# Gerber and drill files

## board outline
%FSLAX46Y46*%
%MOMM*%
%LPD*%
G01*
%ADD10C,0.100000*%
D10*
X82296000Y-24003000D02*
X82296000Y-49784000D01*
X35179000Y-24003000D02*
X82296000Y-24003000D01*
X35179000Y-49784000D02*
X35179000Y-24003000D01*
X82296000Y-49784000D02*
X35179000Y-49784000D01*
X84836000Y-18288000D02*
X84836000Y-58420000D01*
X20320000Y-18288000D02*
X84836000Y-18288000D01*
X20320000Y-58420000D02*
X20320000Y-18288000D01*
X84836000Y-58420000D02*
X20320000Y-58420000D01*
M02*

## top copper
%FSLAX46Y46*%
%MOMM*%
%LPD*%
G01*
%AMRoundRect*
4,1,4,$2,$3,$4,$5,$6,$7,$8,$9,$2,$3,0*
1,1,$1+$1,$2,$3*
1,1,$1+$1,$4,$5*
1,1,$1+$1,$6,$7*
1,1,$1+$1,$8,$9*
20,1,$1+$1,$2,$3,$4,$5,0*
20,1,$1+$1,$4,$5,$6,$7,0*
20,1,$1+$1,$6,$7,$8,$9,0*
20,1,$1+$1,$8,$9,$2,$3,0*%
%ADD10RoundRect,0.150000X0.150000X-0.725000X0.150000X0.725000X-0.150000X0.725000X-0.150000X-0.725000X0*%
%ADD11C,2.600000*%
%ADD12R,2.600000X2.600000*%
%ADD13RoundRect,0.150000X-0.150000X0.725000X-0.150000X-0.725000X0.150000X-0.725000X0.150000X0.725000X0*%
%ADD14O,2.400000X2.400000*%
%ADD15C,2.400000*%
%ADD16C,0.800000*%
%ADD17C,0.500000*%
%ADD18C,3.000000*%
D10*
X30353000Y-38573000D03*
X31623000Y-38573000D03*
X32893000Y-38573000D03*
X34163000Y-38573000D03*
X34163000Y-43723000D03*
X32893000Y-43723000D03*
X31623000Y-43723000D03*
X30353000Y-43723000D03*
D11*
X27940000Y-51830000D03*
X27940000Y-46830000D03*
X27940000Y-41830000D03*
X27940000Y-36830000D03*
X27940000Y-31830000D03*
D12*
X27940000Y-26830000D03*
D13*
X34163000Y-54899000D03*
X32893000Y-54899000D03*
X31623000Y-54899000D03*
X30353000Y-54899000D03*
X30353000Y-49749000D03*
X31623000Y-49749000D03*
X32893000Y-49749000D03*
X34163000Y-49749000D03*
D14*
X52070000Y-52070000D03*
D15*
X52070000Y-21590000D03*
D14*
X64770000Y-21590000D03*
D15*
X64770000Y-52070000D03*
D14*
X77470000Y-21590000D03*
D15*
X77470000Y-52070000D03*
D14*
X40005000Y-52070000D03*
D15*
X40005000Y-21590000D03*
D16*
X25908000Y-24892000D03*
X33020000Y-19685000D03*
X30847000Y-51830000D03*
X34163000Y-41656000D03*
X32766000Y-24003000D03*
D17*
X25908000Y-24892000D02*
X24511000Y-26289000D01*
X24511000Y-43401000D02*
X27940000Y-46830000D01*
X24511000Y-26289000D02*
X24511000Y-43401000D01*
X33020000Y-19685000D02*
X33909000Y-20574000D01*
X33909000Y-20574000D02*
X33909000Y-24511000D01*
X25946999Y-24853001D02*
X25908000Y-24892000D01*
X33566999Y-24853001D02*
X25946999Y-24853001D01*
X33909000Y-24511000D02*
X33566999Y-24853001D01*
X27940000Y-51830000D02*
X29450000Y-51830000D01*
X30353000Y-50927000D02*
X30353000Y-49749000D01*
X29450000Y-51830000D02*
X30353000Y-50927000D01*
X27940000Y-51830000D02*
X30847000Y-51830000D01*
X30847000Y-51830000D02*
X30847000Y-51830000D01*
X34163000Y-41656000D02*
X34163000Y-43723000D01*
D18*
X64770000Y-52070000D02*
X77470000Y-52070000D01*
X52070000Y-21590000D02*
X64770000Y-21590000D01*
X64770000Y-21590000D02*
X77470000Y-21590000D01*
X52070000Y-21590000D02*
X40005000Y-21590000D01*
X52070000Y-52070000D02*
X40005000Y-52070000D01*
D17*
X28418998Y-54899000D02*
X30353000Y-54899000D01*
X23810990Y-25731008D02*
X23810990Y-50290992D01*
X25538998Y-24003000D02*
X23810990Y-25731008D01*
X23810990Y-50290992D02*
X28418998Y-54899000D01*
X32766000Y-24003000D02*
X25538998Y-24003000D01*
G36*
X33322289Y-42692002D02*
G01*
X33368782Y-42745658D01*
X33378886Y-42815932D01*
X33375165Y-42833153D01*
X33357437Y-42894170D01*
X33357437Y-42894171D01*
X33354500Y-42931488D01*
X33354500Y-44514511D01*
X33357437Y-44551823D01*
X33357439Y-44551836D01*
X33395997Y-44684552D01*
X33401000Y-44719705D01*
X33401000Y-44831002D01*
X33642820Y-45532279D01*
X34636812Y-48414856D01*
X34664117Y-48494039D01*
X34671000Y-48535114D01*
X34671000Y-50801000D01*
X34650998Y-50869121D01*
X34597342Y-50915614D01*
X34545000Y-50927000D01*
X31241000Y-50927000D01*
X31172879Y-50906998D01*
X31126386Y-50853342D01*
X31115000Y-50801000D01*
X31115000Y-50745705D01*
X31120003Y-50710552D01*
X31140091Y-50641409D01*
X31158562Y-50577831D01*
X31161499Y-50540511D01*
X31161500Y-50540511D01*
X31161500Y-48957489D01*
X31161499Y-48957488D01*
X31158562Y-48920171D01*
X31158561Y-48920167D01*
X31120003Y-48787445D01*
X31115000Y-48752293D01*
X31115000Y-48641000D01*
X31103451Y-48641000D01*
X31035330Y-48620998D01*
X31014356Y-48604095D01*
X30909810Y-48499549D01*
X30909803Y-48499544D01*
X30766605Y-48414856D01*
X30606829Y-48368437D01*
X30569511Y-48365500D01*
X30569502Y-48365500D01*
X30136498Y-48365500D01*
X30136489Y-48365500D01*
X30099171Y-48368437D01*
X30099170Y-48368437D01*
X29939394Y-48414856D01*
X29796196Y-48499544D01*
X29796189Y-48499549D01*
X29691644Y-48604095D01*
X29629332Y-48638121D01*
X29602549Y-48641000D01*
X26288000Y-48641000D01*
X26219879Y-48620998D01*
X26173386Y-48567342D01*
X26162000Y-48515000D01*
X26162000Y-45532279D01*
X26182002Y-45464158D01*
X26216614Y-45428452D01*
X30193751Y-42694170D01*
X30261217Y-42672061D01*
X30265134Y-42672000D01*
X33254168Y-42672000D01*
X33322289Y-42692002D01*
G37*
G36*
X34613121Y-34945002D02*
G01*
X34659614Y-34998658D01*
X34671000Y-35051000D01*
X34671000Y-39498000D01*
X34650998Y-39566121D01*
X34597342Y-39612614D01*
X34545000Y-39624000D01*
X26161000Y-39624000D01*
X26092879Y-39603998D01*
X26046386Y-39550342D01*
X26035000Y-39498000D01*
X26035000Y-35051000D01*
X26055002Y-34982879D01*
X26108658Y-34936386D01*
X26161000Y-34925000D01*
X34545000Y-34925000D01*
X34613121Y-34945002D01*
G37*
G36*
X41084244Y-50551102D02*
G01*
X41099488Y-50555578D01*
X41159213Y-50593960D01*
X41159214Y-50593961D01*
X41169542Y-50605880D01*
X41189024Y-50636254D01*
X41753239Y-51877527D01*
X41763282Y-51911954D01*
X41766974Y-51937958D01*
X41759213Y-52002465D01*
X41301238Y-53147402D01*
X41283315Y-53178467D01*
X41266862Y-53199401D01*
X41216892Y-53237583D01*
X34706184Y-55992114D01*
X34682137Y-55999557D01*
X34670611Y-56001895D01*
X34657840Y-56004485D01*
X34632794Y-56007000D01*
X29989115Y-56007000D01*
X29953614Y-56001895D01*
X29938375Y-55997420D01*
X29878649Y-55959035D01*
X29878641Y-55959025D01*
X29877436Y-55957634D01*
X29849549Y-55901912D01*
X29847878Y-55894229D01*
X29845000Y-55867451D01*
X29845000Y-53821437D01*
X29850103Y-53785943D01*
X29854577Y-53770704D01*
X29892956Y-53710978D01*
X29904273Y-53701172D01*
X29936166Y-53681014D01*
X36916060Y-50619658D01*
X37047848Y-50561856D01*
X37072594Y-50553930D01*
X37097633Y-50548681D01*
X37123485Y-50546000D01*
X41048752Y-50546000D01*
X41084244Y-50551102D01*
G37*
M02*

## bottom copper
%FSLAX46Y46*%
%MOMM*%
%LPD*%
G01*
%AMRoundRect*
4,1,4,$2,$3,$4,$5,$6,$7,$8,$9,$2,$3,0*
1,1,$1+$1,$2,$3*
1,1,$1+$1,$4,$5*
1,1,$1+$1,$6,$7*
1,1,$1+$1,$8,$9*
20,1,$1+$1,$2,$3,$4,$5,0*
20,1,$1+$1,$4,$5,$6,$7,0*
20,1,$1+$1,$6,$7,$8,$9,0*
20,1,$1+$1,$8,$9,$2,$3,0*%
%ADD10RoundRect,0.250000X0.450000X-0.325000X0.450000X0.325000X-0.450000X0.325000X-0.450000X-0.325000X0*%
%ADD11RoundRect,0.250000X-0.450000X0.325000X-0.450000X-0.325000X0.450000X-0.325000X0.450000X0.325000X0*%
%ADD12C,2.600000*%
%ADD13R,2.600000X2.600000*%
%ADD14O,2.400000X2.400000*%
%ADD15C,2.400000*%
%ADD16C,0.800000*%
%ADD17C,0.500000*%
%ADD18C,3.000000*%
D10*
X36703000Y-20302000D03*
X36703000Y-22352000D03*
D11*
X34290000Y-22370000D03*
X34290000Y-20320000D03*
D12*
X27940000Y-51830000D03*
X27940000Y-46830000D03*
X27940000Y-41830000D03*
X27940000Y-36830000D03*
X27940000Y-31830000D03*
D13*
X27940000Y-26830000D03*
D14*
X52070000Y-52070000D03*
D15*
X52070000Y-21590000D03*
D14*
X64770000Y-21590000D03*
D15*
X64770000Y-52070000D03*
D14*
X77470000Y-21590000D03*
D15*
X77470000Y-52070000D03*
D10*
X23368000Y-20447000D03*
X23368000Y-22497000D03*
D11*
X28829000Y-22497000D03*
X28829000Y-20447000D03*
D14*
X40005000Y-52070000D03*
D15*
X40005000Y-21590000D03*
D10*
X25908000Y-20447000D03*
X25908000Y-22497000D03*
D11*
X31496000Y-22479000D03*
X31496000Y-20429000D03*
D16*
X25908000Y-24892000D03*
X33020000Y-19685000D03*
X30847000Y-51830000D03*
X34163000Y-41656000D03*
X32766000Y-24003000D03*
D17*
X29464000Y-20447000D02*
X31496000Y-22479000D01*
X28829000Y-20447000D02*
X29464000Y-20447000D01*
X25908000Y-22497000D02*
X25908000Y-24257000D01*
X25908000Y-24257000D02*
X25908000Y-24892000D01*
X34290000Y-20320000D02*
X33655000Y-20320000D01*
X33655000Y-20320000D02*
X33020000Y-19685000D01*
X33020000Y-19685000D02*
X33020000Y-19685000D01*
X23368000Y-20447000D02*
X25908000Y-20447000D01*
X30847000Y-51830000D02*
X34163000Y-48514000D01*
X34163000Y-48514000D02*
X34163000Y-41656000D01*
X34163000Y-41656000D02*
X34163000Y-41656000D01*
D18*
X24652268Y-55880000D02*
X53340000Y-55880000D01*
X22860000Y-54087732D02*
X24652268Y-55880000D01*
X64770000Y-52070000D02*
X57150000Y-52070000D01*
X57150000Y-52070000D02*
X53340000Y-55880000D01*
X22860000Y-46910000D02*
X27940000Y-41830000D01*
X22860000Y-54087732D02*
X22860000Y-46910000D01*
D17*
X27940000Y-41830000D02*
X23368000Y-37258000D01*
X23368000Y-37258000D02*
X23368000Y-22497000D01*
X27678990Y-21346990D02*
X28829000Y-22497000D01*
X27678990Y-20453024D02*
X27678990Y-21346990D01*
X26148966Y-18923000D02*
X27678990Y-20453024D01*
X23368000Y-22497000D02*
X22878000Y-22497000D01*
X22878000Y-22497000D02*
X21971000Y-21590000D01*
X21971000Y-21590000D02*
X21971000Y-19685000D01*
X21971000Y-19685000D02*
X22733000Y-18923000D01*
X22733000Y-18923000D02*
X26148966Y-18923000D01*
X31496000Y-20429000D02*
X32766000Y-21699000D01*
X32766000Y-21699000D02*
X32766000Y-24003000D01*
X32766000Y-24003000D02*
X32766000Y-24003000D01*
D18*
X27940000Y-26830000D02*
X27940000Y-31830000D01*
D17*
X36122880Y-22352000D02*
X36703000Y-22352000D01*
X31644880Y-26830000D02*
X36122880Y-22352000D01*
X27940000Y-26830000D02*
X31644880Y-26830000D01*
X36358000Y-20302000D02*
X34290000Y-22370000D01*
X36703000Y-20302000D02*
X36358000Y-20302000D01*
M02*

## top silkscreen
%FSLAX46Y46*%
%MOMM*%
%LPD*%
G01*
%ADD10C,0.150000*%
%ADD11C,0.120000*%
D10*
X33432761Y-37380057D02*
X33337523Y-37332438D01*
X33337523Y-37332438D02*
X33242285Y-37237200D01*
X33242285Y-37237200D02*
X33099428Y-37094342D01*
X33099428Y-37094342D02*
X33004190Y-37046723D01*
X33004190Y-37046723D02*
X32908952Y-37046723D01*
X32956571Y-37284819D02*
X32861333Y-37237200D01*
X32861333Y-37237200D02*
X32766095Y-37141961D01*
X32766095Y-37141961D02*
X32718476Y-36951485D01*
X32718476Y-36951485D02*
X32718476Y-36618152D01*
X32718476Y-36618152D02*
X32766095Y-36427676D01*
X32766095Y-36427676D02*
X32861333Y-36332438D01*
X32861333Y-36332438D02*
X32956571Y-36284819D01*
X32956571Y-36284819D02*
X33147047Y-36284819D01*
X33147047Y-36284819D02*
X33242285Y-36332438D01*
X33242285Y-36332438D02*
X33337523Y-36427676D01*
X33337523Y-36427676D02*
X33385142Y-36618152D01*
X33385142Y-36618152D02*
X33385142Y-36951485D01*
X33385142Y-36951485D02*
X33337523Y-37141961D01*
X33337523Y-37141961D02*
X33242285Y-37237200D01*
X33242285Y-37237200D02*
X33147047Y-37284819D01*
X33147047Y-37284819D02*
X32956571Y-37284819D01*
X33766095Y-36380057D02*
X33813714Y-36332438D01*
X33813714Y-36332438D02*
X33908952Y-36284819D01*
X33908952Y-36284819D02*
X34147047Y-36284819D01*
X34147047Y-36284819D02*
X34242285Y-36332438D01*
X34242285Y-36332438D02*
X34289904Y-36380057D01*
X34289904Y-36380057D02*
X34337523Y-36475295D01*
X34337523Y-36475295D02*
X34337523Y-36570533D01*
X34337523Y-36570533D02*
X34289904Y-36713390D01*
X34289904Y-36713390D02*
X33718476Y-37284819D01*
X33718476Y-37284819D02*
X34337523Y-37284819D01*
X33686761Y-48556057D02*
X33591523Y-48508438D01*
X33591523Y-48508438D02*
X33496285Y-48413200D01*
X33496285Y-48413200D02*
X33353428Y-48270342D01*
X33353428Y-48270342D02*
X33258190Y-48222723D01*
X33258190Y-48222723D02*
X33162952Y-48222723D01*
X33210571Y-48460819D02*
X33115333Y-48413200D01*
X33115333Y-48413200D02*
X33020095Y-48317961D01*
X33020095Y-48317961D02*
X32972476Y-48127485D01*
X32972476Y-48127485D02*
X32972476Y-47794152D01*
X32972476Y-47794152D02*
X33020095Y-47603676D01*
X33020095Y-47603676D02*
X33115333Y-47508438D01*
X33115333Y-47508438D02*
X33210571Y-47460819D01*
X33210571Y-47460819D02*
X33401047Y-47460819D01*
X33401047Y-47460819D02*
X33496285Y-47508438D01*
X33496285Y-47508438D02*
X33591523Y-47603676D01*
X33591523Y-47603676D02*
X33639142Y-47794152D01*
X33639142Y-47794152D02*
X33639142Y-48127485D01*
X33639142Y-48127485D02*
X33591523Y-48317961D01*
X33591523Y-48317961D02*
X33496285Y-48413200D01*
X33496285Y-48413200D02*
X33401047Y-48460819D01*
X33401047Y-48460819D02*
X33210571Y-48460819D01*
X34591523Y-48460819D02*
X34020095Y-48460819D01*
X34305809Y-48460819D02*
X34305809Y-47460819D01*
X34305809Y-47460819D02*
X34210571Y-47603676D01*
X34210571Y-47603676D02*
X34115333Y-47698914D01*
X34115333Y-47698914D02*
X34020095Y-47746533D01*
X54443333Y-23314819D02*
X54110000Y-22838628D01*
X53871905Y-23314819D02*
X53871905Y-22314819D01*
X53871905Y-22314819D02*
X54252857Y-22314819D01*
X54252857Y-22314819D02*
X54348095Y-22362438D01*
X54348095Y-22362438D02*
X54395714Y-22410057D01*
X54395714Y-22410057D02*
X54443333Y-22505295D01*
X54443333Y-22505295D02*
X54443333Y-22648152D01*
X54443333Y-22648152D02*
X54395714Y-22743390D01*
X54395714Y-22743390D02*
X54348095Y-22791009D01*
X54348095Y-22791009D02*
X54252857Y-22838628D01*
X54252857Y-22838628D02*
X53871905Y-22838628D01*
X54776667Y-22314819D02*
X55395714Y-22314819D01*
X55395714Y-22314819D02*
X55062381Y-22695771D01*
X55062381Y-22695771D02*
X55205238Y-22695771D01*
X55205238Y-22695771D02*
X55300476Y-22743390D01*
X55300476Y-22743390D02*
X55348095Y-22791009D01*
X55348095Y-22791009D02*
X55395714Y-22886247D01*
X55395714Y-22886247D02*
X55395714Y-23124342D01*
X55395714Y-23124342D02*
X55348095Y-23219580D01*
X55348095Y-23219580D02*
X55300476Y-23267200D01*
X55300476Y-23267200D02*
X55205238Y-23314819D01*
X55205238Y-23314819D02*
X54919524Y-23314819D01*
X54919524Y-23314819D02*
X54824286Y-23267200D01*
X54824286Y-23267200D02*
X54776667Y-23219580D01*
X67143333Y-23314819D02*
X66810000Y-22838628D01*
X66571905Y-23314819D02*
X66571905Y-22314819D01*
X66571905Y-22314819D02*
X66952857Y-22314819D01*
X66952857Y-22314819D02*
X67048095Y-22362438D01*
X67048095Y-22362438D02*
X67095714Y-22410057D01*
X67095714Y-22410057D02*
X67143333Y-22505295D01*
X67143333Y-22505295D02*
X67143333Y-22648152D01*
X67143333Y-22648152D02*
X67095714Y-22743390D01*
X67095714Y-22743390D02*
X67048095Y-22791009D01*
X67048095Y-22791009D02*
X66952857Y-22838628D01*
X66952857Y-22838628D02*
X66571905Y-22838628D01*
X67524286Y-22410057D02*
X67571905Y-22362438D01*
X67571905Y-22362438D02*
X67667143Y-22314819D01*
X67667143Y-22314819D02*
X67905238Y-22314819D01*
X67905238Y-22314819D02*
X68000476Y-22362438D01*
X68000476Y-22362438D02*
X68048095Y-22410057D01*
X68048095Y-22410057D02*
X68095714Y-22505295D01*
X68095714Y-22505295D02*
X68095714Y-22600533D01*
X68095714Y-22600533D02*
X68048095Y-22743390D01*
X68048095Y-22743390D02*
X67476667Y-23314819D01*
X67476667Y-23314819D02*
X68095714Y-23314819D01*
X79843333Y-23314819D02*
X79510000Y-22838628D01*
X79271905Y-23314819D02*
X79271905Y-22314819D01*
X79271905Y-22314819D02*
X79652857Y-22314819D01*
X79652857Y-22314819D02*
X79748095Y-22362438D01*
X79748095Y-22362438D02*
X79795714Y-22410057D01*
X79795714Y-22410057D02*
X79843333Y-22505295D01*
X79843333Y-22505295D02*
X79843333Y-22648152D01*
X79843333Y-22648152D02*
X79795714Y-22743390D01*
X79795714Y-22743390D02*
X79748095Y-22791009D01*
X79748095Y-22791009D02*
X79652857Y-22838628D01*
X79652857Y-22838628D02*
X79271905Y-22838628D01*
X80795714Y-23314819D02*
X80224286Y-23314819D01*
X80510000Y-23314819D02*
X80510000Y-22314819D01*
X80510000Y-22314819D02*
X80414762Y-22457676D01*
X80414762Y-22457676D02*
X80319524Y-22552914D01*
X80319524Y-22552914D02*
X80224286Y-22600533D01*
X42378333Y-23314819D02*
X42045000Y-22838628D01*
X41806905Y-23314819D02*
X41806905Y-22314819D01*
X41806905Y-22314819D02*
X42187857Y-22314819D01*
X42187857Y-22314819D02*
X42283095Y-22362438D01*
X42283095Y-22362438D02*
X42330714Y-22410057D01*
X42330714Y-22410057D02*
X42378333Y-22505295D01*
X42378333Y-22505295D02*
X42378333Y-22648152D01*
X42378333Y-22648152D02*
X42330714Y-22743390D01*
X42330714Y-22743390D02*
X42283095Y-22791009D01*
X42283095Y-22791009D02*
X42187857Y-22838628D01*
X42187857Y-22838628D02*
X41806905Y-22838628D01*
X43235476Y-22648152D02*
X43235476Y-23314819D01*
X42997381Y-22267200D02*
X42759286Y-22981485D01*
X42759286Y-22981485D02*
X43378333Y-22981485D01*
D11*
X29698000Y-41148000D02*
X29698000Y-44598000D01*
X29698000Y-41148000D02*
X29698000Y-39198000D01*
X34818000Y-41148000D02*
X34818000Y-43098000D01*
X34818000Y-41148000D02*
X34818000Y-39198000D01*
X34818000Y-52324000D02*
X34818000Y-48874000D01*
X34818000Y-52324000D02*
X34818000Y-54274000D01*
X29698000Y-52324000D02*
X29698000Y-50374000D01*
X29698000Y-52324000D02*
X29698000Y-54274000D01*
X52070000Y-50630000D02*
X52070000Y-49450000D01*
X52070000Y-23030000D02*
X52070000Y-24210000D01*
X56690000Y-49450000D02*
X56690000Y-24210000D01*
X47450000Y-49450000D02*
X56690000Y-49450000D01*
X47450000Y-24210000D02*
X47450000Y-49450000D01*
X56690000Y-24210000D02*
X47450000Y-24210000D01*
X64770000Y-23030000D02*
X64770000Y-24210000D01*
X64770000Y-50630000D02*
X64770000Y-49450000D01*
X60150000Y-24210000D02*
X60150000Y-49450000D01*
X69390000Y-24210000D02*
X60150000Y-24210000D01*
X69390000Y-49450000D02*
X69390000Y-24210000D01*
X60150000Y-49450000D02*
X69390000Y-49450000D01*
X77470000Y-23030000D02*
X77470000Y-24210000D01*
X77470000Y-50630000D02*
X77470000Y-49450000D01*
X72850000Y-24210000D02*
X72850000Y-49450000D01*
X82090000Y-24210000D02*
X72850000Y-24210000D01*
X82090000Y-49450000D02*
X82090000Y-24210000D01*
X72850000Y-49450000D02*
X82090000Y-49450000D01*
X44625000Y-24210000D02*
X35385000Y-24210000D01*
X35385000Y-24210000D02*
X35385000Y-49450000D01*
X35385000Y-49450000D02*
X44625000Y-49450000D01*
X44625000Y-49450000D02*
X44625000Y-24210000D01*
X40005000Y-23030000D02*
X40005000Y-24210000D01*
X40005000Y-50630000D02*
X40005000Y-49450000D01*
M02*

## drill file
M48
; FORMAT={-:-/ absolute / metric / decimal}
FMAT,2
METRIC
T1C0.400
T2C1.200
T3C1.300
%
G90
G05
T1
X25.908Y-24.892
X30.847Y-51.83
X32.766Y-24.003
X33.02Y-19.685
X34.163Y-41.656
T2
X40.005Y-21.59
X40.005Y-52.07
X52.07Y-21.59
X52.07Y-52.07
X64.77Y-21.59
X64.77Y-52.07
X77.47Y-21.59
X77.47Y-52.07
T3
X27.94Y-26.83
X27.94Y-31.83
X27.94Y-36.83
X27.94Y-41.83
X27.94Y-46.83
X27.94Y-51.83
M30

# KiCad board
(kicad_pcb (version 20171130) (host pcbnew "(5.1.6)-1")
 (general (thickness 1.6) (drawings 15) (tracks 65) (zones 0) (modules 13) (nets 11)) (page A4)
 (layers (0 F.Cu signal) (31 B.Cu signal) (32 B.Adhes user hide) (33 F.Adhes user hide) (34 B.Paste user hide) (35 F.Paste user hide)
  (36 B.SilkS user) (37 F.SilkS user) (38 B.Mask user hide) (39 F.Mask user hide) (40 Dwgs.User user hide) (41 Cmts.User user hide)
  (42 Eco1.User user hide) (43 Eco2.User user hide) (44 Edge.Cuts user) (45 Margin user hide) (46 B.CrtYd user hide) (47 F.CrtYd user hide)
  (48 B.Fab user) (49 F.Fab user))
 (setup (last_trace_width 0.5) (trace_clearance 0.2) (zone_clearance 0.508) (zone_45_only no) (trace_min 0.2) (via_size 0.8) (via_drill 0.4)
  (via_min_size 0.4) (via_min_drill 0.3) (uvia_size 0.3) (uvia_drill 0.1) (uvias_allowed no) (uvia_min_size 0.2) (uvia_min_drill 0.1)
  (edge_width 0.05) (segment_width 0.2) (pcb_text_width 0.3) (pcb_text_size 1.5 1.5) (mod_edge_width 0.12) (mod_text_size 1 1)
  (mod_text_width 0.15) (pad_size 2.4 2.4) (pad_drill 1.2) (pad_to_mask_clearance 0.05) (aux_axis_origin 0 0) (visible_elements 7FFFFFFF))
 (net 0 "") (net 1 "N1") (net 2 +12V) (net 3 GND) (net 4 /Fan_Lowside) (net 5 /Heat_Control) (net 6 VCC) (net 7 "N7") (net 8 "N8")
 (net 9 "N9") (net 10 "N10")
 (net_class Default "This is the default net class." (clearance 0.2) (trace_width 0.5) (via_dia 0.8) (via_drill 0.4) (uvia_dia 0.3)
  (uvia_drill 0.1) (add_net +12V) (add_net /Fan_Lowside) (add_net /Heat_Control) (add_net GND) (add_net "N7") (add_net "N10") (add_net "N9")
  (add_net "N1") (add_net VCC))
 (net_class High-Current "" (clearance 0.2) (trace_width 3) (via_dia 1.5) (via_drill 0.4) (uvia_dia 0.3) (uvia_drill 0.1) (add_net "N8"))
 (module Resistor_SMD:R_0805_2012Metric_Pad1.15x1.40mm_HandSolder (layer B.Cu) (at 36.703 21.327 90)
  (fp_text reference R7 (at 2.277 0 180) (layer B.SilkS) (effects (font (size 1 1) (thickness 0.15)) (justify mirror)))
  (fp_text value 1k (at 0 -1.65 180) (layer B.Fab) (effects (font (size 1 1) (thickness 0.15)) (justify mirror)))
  (pad 2 smd roundrect (at 1.025 0 90) (size 1.15 1.4) (layers B.Cu B.Paste B.Mask) (roundrect_rratio 0.217391) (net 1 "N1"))
  (pad 1 smd roundrect (at -1.025 0 90) (size 1.15 1.4) (layers B.Cu B.Paste B.Mask) (roundrect_rratio 0.217391) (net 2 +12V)))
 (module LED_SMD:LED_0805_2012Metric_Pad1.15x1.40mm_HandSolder (layer B.Cu) (at 34.29 21.345 270)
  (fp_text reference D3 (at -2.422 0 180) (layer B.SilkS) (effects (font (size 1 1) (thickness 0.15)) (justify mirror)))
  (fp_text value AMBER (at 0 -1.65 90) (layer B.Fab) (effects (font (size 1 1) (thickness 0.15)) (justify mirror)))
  (pad 2 smd roundrect (at 1.025 0 270) (size 1.15 1.4) (layers B.Cu B.Paste B.Mask) (roundrect_rratio 0.217391) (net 1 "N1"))
  (pad 1 smd roundrect (at -1.025 0 270) (size 1.15 1.4) (layers B.Cu B.Paste B.Mask) (roundrect_rratio 0.217391) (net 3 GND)))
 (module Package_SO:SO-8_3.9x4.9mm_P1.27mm (layer F.Cu) (at 32.258 41.148 90)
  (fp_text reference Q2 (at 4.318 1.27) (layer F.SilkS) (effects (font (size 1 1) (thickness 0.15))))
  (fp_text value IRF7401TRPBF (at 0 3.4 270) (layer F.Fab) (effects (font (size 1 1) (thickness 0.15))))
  (fp_line (start 0 -2.56) (end -3.45 -2.56) (layer F.SilkS) (width 0.12))
  (fp_line (start 0 -2.56) (end 1.95 -2.56) (layer F.SilkS) (width 0.12))
  (fp_line (start 0 2.56) (end -1.95 2.56) (layer F.SilkS) (width 0.12))
  (fp_line (start 0 2.56) (end 1.95 2.56) (layer F.SilkS) (width 0.12))
  (pad 3 smd roundrect (at 2.575 -1.905 90) (size 1.75 0.6) (layers F.Cu F.Paste F.Mask) (roundrect_rratio 0.25) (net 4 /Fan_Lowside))
  (pad 3 smd roundrect (at 2.575 -0.635 90) (size 1.75 0.6) (layers F.Cu F.Paste F.Mask) (roundrect_rratio 0.25) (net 4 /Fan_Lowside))
  (pad 3 smd roundrect (at 2.575 0.635 90) (size 1.75 0.6) (layers F.Cu F.Paste F.Mask) (roundrect_rratio 0.25) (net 4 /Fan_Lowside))
  (pad 3 smd roundrect (at 2.575 1.905 90) (size 1.75 0.6) (layers F.Cu F.Paste F.Mask) (roundrect_rratio 0.25) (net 4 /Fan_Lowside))
  (pad 1 smd roundrect (at -2.575 1.905 90) (size 1.75 0.6) (layers F.Cu F.Paste F.Mask) (roundrect_rratio 0.25) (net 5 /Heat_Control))
  (pad 2 smd roundrect (at -2.575 0.635 90) (size 1.75 0.6) (layers F.Cu F.Paste F.Mask) (roundrect_rratio 0.25) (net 3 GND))
  (pad 2 smd roundrect (at -2.575 -0.635 90) (size 1.75 0.6) (layers F.Cu F.Paste F.Mask) (roundrect_rratio 0.25) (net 3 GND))
  (pad 2 smd roundrect (at -2.575 -1.905 90) (size 1.75 0.6) (layers F.Cu F.Paste F.Mask) (roundrect_rratio 0.25) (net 3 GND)))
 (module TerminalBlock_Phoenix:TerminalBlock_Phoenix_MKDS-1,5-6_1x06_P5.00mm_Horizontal (layer B.Cu) (at 27.94 26.83 270)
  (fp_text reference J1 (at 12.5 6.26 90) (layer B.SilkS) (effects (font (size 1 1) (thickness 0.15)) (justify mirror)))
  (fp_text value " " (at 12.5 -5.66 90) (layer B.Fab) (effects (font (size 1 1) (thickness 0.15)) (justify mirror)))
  (pad 6 thru_hole circle (at 25 0 270) (size 2.6 2.6) (drill 1.3) (layers *.Cu *.Mask) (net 5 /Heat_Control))
  (pad 5 thru_hole circle (at 20 0 270) (size 2.6 2.6) (drill 1.3) (layers *.Cu *.Mask) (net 3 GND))
  (pad 4 thru_hole circle (at 15 0 270) (size 2.6 2.6) (drill 1.3) (layers *.Cu *.Mask) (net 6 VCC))
  (pad 3 thru_hole circle (at 10 0 270) (size 2.6 2.6) (drill 1.3) (layers *.Cu *.Mask) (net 4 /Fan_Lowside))
  (pad 2 thru_hole circle (at 5 0 270) (size 2.6 2.6) (drill 1.3) (layers *.Cu *.Mask) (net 2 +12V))
  (pad 1 thru_hole rect (at 0 0 270) (size 2.6 2.6) (drill 1.3) (layers *.Cu *.Mask) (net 2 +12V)))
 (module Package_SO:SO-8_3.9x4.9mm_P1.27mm (layer F.Cu) (at 32.258 52.324 270)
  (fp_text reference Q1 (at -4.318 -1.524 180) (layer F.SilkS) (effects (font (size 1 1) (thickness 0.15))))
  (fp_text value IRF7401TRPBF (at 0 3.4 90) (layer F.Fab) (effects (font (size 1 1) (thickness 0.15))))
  (fp_line (start 0 -2.56) (end -3.45 -2.56) (layer F.SilkS) (width 0.12))
  (fp_line (start 0 -2.56) (end 1.95 -2.56) (layer F.SilkS) (width 0.12))
  (fp_line (start 0 2.56) (end -1.95 2.56) (layer F.SilkS) (width 0.12))
  (fp_line (start 0 2.56) (end 1.95 2.56) (layer F.SilkS) (width 0.12))
  (pad 3 smd roundrect (at 2.575 -1.905 270) (size 1.75 0.6) (layers F.Cu F.Paste F.Mask) (roundrect_rratio 0.25) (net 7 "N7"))
  (pad 3 smd roundrect (at 2.575 -0.635 270) (size 1.75 0.6) (layers F.Cu F.Paste F.Mask) (roundrect_rratio 0.25) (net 7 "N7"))
  (pad 3 smd roundrect (at 2.575 0.635 270) (size 1.75 0.6) (layers F.Cu F.Paste F.Mask) (roundrect_rratio 0.25) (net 7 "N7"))
  (pad 3 smd roundrect (at 2.575 1.905 270) (size 1.75 0.6) (layers F.Cu F.Paste F.Mask) (roundrect_rratio 0.25) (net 7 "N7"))
  (pad 1 smd roundrect (at -2.575 1.905 270) (size 1.75 0.6) (layers F.Cu F.Paste F.Mask) (roundrect_rratio 0.25) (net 5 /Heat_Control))
  (pad 2 smd roundrect (at -2.575 0.635 270) (size 1.75 0.6) (layers F.Cu F.Paste F.Mask) (roundrect_rratio 0.25) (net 3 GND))
  (pad 2 smd roundrect (at -2.575 -0.635 270) (size 1.75 0.6) (layers F.Cu F.Paste F.Mask) (roundrect_rratio 0.25) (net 3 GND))
  (pad 2 smd roundrect (at -2.575 -1.905 270) (size 1.75 0.6) (layers F.Cu F.Paste F.Mask) (roundrect_rratio 0.25) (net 3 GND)))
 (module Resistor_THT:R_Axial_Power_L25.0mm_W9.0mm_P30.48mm (layer F.Cu) (at 52.07 21.59 270)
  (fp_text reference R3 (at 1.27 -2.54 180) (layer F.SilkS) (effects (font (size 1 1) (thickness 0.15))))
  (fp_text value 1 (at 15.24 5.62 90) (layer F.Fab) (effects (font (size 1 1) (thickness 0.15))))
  (fp_line (start 29.04 0) (end 27.86 0) (layer F.SilkS) (width 0.12))
  (fp_line (start 1.44 0) (end 2.62 0) (layer F.SilkS) (width 0.12))
  (fp_line (start 27.86 -4.62) (end 2.62 -4.62) (layer F.SilkS) (width 0.12))
  (fp_line (start 27.86 4.62) (end 27.86 -4.62) (layer F.SilkS) (width 0.12))
  (fp_line (start 2.62 4.62) (end 27.86 4.62) (layer F.SilkS) (width 0.12))
  (fp_line (start 2.62 -4.62) (end 2.62 4.62) (layer F.SilkS) (width 0.12))
  (pad 2 thru_hole oval (at 30.48 0 270) (size 2.4 2.4) (drill 1.2) (layers *.Cu *.Mask) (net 7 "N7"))
  (pad 1 thru_hole circle (at 0 0 270) (size 2.4 2.4) (drill 1.2) (layers *.Cu *.Mask) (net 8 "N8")))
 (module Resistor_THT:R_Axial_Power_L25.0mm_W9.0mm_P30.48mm (layer F.Cu) (at 64.77 52.07 90)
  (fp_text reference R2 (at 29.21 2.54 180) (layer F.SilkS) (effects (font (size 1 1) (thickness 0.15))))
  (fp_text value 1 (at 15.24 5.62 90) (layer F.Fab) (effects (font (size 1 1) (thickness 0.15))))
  (fp_line (start 29.04 0) (end 27.86 0) (layer F.SilkS) (width 0.12))
  (fp_line (start 1.44 0) (end 2.62 0) (layer F.SilkS) (width 0.12))
  (fp_line (start 27.86 -4.62) (end 2.62 -4.62) (layer F.SilkS) (width 0.12))
  (fp_line (start 27.86 4.62) (end 27.86 -4.62) (layer F.SilkS) (width 0.12))
  (fp_line (start 2.62 4.62) (end 27.86 4.62) (layer F.SilkS) (width 0.12))
  (fp_line (start 2.62 -4.62) (end 2.62 4.62) (layer F.SilkS) (width 0.12))
  (pad 2 thru_hole oval (at 30.48 0 90) (size 2.4 2.4) (drill 1.2) (layers *.Cu *.Mask) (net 8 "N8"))
  (pad 1 thru_hole circle (at 0 0 90) (size 2.4 2.4) (drill 1.2) (layers *.Cu *.Mask) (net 6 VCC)))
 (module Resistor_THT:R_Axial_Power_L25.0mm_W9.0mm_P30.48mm (layer F.Cu) (at 77.47 52.07 90)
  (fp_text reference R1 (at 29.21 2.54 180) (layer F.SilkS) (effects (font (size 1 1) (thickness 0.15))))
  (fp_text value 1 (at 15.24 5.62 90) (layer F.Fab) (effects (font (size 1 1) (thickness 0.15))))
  (fp_line (start 29.04 0) (end 27.86 0) (layer F.SilkS) (width 0.12))
  (fp_line (start 1.44 0) (end 2.62 0) (layer F.SilkS) (width 0.12))
  (fp_line (start 27.86 -4.62) (end 2.62 -4.62) (layer F.SilkS) (width 0.12))
  (fp_line (start 27.86 4.62) (end 27.86 -4.62) (layer F.SilkS) (width 0.12))
  (fp_line (start 2.62 4.62) (end 27.86 4.62) (layer F.SilkS) (width 0.12))
  (fp_line (start 2.62 -4.62) (end 2.62 4.62) (layer F.SilkS) (width 0.12))
  (pad 2 thru_hole oval (at 30.48 0 90) (size 2.4 2.4) (drill 1.2) (layers *.Cu *.Mask) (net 8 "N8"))
  (pad 1 thru_hole circle (at 0 0 90) (size 2.4 2.4) (drill 1.2) (layers *.Cu *.Mask) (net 6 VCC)))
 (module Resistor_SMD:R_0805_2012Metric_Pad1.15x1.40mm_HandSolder (layer B.Cu) (at 23.368 21.472 90)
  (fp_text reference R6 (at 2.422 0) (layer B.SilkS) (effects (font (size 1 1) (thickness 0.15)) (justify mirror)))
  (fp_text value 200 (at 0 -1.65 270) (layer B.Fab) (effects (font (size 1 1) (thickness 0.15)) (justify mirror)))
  (pad 2 smd roundrect (at 1.025 0 90) (size 1.15 1.4) (layers B.Cu B.Paste B.Mask) (roundrect_rratio 0.217391) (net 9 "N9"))
  (pad 1 smd roundrect (at -1.025 0 90) (size 1.15 1.4) (layers B.Cu B.Paste B.Mask) (roundrect_rratio 0.217391) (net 6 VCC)))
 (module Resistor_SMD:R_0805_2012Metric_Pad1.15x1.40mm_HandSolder (layer B.Cu) (at 28.829 21.472 270)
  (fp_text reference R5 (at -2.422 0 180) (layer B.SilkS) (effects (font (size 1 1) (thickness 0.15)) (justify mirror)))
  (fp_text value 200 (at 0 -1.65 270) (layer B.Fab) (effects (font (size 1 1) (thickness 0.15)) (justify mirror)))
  (pad 2 smd roundrect (at 1.025 0 270) (size 1.15 1.4) (layers B.Cu B.Paste B.Mask) (roundrect_rratio 0.217391) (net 6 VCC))
  (pad 1 smd roundrect (at -1.025 0 270) (size 1.15 1.4) (layers B.Cu B.Paste B.Mask) (roundrect_rratio 0.217391) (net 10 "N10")))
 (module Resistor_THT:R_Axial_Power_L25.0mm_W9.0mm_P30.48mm (layer F.Cu) (at 40.005 21.59 270)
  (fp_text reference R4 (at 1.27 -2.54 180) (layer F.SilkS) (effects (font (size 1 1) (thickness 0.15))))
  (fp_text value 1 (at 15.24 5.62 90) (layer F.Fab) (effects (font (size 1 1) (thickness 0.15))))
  (fp_line (start 2.62 -4.62) (end 2.62 4.62) (layer F.SilkS) (width 0.12))
  (fp_line (start 2.62 4.62) (end 27.86 4.62) (layer F.SilkS) (width 0.12))
  (fp_line (start 27.86 4.62) (end 27.86 -4.62) (layer F.SilkS) (width 0.12))
  (fp_line (start 27.86 -4.62) (end 2.62 -4.62) (layer F.SilkS) (width 0.12))
  (fp_line (start 1.44 0) (end 2.62 0) (layer F.SilkS) (width 0.12))
  (fp_line (start 29.04 0) (end 27.86 0) (layer F.SilkS) (width 0.12))
  (pad 2 thru_hole oval (at 30.48 0 270) (size 2.4 2.4) (drill 1.2) (layers *.Cu *.Mask) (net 7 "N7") (zone_connect 2))
  (pad 1 thru_hole circle (at 0 0 270) (size 2.4 2.4) (drill 1.2) (layers *.Cu *.Mask) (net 8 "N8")))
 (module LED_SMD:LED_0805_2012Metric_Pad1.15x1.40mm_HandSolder (layer B.Cu) (at 25.908 21.472 90)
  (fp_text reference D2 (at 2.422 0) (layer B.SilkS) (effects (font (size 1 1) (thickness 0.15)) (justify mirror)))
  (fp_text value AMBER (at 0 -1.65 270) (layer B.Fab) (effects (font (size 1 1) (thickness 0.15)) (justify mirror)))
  (pad 2 smd roundrect (at 1.025 0 90) (size 1.15 1.4) (layers B.Cu B.Paste B.Mask) (roundrect_rratio 0.217391) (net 9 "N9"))
  (pad 1 smd roundrect (at -1.025 0 90) (size 1.15 1.4) (layers B.Cu B.Paste B.Mask) (roundrect_rratio 0.217391) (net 3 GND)))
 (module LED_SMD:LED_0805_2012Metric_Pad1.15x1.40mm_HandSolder (layer B.Cu) (at 31.496 21.454 270)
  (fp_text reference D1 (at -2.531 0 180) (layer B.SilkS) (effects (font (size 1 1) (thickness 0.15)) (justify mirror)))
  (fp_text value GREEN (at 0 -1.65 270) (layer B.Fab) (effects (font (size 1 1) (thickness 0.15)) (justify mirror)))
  (pad 2 smd roundrect (at 1.025 0 270) (size 1.15 1.4) (layers B.Cu B.Paste B.Mask) (roundrect_rratio 0.217391) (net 10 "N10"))
  (pad 1 smd roundrect (at -1.025 0 270) (size 1.15 1.4) (layers B.Cu B.Paste B.Mask) (roundrect_rratio 0.217391) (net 7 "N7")))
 (gr_line (start 82.296 24.003) (end 82.296 49.784) (layer Edge.Cuts) (width 0.1))
 (gr_line (start 35.179 24.003) (end 82.296 24.003) (layer Edge.Cuts) (width 0.1))
 (gr_line (start 35.179 49.784) (end 35.179 24.003) (layer Edge.Cuts) (width 0.1))
 (gr_line (start 82.296 49.784) (end 35.179 49.784) (layer Edge.Cuts) (width 0.1))
 (gr_line (start 84.836 18.288) (end 84.836 58.42) (layer Edge.Cuts) (width 0.1))
 (gr_line (start 20.32 18.288) (end 84.836 18.288) (layer Edge.Cuts) (width 0.1))
 (gr_line (start 20.32 58.42) (end 20.32 18.288) (layer Edge.Cuts) (width 0.1))
 (gr_line (start 84.836 58.42) (end 20.32 58.42) (layer Edge.Cuts) (width 0.1))
 (segment (start 29.464 20.447) (end 31.496 22.479) (width 0.5) (layer B.Cu) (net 10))
 (segment (start 28.829 20.447) (end 29.464 20.447) (width 0.5) (layer B.Cu) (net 10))
 (via (at 25.908 24.892) (size 0.8) (drill 0.4) (layers F.Cu B.Cu) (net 3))
 (segment (start 25.908 22.497) (end 25.908 24.257) (width 0.5) (layer B.Cu) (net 3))
 (segment (start 25.908 24.892) (end 24.511 26.289) (width 0.5) (layer F.Cu) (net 3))
 (segment (start 25.908 24.257) (end 25.908 24.892) (width 0.5) (layer B.Cu) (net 3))
 (segment (start 24.511 43.401) (end 27.94 46.83) (width 0.5) (layer F.Cu) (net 3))
 (segment (start 24.511 26.289) (end 24.511 43.401) (width 0.5) (layer F.Cu) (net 3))
 (segment (start 34.29 20.32) (end 33.655 20.32) (width 0.5) (layer B.Cu) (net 3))
 (segment (start 33.655 20.32) (end 33.02 19.685) (width 0.5) (layer B.Cu) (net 3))
 (segment (start 33.02 19.685) (end 33.02 19.685) (width 0.5) (layer B.Cu) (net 3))
 (via (at 33.02 19.685) (size 0.8) (drill 0.4) (layers F.Cu B.Cu) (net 3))
 (segment (start 33.02 19.685) (end 33.909 20.574) (width 0.5) (layer F.Cu) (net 3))
 (segment (start 33.909 20.574) (end 33.909 24.511) (width 0.5) (layer F.Cu) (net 3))
 (segment (start 25.946999 24.853001) (end 25.908 24.892) (width 0.5) (layer F.Cu) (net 3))
 (segment (start 33.566999 24.853001) (end 25.946999 24.853001) (width 0.5) (layer F.Cu) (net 3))
 (segment (start 33.909 24.511) (end 33.566999 24.853001) (width 0.5) (layer F.Cu) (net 3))
 (segment (start 23.368 20.447) (end 25.908 20.447) (width 0.5) (layer B.Cu) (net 9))
 (segment (start 27.94 51.83) (end 29.45 51.83) (width 0.5) (layer F.Cu) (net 5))
 (segment (start 30.353 50.927) (end 30.353 49.749) (width 0.5) (layer F.Cu) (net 5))
 (segment (start 29.45 51.83) (end 30.353 50.927) (width 0.5) (layer F.Cu) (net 5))
 (segment (start 27.94 51.83) (end 30.847 51.83) (width 0.5) (layer F.Cu) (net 5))
 (segment (start 30.847 51.83) (end 30.847 51.83) (width 0.5) (layer F.Cu) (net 5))
 (via (at 30.847 51.83) (size 0.8) (drill 0.4) (layers F.Cu B.Cu) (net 5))
 (segment (start 30.847 51.83) (end 34.163 48.514) (width 0.5) (layer B.Cu) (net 5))
 (segment (start 34.163 48.514) (end 34.163 41.656) (width 0.5) (layer B.Cu) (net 5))
 (segment (start 34.163 41.656) (end 34.163 41.656) (width 0.5) (layer B.Cu) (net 5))
 (via (at 34.163 41.656) (size 0.8) (drill 0.4) (layers F.Cu B.Cu) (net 5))
 (segment (start 34.163 41.656) (end 34.163 43.723) (width 0.5) (layer F.Cu) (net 5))
 (segment (start 64.77 52.07) (end 77.47 52.07) (width 3) (layer F.Cu) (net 6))
 (segment (start 24.652268 55.88) (end 53.34 55.88) (width 3) (layer B.Cu) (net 6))
 (segment (start 22.86 54.087732) (end 24.652268 55.88) (width 3) (layer B.Cu) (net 6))
 (segment (start 64.77 52.07) (end 57.15 52.07) (width 3) (layer B.Cu) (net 6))
 (segment (start 57.15 52.07) (end 53.34 55.88) (width 3) (layer B.Cu) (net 6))
 (segment (start 22.86 46.91) (end 27.94 41.83) (width 3) (layer B.Cu) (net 6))
 (segment (start 22.86 54.087732) (end 22.86 46.91) (width 3) (layer B.Cu) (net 6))
 (segment (start 27.94 41.83) (end 23.368 37.258) (width 0.5) (layer B.Cu) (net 6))
 (segment (start 23.368 37.258) (end 23.368 22.497) (width 0.5) (layer B.Cu) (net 6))
 (segment (start 27.67899 21.34699) (end 28.829 22.497) (width 0.5) (layer B.Cu) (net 6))
 (segment (start 27.67899 20.453024) (end 27.67899 21.34699) (width 0.5) (layer B.Cu) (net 6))
 (segment (start 26.148966 18.923) (end 27.67899 20.453024) (width 0.5) (layer B.Cu) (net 6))
 (segment (start 23.368 22.497) (end 22.878 22.497) (width 0.5) (layer B.Cu) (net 6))
 (segment (start 22.878 22.497) (end 21.971 21.59) (width 0.5) (layer B.Cu) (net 6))
 (segment (start 21.971 21.59) (end 21.971 19.685) (width 0.5) (layer B.Cu) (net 6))
 (segment (start 21.971 19.685) (end 22.733 18.923) (width 0.5) (layer B.Cu) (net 6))
 (segment (start 22.733 18.923) (end 26.148966 18.923) (width 0.5) (layer B.Cu) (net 6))
 (segment (start 52.07 21.59) (end 64.77 21.59) (width 3) (layer F.Cu) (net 8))
 (segment (start 64.77 21.59) (end 77.47 21.59) (width 3) (layer F.Cu) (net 8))
 (segment (start 52.07 21.59) (end 40.005 21.59) (width 3) (layer F.Cu) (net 8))
 (segment (start 52.07 52.07) (end 40.005 52.07) (width 3) (layer F.Cu) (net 7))
 (segment (start 31.496 20.429) (end 32.766 21.699) (width 0.5) (layer B.Cu) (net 7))
 (segment (start 32.766 21.699) (end 32.766 24.003) (width 0.5) (layer B.Cu) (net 7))
 (segment (start 32.766 24.003) (end 32.766 24.003) (width 0.5) (layer B.Cu) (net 7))
 (via (at 32.766 24.003) (size 0.8) (drill 0.4) (layers F.Cu B.Cu) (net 7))
 (segment (start 28.418998 54.899) (end 30.353 54.899) (width 0.5) (layer F.Cu) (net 7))
 (segment (start 23.81099 25.731008) (end 23.81099 50.290992) (width 0.5) (layer F.Cu) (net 7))
 (segment (start 25.538998 24.003) (end 23.81099 25.731008) (width 0.5) (layer F.Cu) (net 7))
 (segment (start 23.81099 50.290992) (end 28.418998 54.899) (width 0.5) (layer F.Cu) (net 7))
 (segment (start 32.766 24.003) (end 25.538998 24.003) (width 0.5) (layer F.Cu) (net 7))
 (segment (start 27.94 26.83) (end 27.94 31.83) (width 3) (layer B.Cu) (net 2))
 (segment (start 36.12288 22.352) (end 36.703 22.352) (width 0.5) (layer B.Cu) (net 2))
 (segment (start 31.64488 26.83) (end 36.12288 22.352) (width 0.5) (layer B.Cu) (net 2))
 (segment (start 27.94 26.83) (end 31.64488 26.83) (width 0.5) (layer B.Cu) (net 2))
 (segment (start 36.358 20.302) (end 34.29 22.37) (width 0.5) (layer B.Cu) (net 1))
 (segment (start 36.703 20.302) (end 36.358 20.302) (width 0.5) (layer B.Cu) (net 1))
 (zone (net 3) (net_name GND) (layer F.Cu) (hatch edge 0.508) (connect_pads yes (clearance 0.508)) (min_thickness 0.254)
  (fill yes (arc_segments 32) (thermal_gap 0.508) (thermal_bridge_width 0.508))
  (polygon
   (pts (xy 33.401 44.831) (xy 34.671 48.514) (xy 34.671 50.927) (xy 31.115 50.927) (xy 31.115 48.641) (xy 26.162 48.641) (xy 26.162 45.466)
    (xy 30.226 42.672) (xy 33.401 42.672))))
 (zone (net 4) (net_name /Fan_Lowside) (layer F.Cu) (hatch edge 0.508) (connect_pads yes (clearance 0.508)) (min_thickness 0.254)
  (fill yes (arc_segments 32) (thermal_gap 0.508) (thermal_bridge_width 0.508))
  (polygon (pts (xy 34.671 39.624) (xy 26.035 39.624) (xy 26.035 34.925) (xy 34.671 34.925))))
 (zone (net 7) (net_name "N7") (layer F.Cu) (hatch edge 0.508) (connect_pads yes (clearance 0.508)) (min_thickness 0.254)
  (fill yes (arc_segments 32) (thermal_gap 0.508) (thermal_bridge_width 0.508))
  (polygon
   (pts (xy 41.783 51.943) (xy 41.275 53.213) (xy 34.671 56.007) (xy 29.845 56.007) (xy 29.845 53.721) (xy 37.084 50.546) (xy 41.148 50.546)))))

